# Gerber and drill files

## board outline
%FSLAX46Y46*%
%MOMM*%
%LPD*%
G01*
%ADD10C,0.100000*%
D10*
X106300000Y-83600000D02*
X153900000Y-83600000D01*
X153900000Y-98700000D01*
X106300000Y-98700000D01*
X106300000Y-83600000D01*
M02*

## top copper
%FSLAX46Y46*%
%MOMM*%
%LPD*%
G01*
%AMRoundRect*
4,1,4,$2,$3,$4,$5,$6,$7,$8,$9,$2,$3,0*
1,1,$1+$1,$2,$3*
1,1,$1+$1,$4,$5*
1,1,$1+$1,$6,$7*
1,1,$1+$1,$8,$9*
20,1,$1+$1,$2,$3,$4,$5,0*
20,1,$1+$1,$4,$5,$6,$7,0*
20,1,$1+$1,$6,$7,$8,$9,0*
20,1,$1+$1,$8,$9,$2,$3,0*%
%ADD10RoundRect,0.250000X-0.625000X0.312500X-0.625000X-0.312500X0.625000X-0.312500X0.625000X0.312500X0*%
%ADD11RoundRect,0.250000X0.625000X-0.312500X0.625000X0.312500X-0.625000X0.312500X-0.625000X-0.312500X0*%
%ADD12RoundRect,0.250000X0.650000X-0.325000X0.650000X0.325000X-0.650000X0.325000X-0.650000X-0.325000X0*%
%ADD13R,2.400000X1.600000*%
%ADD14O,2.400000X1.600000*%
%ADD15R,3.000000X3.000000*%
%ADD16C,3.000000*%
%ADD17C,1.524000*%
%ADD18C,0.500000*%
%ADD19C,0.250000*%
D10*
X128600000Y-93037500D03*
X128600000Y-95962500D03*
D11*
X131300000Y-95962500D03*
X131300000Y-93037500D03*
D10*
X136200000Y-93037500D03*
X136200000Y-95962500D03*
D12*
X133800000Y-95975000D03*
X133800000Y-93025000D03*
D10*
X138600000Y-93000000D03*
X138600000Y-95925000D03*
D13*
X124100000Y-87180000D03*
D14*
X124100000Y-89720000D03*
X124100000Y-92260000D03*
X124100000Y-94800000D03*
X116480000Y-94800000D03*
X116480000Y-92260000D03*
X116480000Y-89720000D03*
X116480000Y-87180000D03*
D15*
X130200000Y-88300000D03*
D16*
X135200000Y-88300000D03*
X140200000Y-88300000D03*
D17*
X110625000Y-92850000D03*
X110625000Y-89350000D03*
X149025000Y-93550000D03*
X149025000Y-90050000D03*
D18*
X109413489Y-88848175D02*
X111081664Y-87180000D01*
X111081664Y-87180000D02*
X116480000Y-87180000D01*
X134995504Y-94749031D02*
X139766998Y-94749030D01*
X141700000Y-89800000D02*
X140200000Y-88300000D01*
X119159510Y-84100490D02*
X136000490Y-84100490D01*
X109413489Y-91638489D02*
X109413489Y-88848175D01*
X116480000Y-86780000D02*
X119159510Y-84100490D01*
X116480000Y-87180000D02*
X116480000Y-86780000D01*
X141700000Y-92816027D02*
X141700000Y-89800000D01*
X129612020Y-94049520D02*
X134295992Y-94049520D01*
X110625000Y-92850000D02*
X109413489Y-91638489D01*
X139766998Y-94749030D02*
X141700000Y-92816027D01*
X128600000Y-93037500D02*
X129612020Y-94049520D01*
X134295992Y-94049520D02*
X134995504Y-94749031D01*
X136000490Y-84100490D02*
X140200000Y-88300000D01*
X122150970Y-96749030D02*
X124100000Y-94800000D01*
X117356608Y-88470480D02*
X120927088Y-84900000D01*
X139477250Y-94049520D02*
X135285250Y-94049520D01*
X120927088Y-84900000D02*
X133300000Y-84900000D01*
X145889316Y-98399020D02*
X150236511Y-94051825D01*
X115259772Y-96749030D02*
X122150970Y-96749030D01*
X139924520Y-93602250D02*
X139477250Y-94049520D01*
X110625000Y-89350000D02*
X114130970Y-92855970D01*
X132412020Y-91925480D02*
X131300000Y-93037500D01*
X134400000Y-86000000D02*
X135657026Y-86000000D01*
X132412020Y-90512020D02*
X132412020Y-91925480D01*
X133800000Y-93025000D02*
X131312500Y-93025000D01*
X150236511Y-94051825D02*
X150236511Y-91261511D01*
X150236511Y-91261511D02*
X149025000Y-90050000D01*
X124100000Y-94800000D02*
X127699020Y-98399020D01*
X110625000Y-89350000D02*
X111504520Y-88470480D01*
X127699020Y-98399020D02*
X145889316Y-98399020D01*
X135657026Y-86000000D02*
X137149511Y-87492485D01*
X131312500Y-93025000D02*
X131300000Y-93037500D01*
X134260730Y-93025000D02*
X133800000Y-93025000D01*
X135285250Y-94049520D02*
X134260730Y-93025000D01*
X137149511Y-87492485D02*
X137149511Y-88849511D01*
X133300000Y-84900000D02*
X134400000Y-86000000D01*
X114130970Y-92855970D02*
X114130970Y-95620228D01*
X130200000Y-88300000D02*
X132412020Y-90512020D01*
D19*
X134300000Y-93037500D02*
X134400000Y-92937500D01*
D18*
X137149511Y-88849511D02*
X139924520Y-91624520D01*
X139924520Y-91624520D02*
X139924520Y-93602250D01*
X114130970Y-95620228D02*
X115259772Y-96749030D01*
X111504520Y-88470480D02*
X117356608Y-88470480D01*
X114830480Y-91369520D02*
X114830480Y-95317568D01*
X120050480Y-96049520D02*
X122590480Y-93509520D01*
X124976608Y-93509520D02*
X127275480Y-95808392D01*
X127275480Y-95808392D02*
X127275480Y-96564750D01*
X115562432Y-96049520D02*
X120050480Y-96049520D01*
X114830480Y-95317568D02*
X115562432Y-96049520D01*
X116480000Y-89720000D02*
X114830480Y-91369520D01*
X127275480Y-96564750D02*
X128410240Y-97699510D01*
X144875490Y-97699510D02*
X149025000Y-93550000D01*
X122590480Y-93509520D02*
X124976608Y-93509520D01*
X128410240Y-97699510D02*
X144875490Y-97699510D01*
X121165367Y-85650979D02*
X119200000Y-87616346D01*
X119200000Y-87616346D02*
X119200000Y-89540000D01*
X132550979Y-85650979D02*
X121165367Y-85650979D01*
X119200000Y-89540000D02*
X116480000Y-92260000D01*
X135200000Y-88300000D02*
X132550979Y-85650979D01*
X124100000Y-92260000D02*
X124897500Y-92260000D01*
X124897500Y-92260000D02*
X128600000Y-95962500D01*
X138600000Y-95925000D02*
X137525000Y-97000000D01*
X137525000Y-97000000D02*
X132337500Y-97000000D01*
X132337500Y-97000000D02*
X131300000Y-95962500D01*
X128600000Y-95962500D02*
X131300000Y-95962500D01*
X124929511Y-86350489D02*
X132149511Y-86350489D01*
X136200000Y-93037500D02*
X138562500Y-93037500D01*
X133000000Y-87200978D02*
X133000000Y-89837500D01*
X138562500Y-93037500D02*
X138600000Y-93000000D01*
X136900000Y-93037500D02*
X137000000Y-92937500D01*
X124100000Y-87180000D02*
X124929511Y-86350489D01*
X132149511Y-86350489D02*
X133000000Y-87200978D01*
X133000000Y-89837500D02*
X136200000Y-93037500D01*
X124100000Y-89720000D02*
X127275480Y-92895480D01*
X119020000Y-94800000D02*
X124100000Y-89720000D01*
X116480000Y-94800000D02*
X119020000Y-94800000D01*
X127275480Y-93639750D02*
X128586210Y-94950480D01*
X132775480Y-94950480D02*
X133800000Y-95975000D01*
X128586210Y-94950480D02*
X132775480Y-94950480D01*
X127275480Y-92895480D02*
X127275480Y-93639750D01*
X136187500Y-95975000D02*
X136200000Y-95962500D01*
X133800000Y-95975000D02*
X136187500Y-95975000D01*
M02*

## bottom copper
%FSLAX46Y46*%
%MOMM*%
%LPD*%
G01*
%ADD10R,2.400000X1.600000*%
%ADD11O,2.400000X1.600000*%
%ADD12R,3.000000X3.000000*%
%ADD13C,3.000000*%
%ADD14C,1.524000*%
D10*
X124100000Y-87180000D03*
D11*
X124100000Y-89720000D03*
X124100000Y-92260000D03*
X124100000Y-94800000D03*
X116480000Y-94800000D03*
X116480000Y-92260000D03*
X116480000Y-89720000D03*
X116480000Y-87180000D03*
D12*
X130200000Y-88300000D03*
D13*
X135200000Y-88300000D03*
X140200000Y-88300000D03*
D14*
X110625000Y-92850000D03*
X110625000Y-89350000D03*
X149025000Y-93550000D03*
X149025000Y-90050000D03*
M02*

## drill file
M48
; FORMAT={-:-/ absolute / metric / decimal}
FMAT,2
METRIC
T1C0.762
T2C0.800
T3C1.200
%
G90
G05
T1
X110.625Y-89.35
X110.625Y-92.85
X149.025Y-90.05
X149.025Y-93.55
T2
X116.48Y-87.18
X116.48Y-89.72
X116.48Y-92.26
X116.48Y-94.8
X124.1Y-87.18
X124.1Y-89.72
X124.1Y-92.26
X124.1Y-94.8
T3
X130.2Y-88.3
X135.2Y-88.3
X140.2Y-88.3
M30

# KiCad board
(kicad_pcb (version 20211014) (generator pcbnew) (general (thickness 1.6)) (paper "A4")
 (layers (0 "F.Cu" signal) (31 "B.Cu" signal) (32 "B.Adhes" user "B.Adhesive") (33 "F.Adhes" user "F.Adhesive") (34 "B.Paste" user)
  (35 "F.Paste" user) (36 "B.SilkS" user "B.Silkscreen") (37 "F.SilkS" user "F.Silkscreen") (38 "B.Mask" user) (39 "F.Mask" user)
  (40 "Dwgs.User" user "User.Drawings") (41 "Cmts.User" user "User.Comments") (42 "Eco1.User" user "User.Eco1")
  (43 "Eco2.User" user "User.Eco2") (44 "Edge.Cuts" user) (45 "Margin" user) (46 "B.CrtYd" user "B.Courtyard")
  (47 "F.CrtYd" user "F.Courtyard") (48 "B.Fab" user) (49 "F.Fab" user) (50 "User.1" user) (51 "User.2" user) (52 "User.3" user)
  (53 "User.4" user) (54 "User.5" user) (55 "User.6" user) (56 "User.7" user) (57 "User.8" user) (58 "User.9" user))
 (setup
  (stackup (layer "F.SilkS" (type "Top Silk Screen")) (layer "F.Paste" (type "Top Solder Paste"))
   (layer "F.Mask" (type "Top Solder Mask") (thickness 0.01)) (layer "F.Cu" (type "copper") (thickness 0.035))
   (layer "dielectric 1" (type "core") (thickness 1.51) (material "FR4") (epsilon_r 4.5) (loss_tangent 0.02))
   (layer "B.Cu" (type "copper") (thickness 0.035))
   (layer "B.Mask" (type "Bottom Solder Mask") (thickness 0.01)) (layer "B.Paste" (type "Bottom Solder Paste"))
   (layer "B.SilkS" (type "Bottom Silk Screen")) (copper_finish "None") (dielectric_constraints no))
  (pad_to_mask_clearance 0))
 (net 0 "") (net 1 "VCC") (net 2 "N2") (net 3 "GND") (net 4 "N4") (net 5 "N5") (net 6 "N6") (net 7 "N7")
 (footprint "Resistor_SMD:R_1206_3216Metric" (layer "F.Cu") (at 128.6 94.5 -90)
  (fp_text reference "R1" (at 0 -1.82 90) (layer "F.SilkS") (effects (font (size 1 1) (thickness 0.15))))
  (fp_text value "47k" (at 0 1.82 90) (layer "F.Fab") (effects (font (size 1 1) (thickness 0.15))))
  (pad "1" smd roundrect (at -1.4625 0 270) (size 1.125 1.75) (layers "F.Cu" "F.Paste" "F.Mask") (roundrect_rratio 0.2222222222)
   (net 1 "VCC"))
  (pad "2" smd roundrect (at 1.4625 0 270) (size 1.125 1.75) (layers "F.Cu" "F.Paste" "F.Mask") (roundrect_rratio 0.2222222222) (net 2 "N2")))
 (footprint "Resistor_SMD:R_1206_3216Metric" (layer "F.Cu") (at 131.3 94.5 90)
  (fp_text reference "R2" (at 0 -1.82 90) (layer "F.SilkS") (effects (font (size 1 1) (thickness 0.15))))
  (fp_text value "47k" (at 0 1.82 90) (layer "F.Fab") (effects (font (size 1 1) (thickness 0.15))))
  (pad "1" smd roundrect (at -1.4625 0 90) (size 1.125 1.75) (layers "F.Cu" "F.Paste" "F.Mask") (roundrect_rratio 0.2222222222) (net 2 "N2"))
  (pad "2" smd roundrect (at 1.4625 0 90) (size 1.125 1.75) (layers "F.Cu" "F.Paste" "F.Mask") (roundrect_rratio 0.2222222222) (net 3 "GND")))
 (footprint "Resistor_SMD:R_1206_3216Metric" (layer "F.Cu") (at 136.2 94.5 -90)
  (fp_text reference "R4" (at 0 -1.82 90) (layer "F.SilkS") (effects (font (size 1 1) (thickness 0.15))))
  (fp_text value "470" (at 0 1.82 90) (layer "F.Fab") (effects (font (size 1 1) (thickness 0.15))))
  (pad "1" smd roundrect (at -1.4625 0 270) (size 1.125 1.75) (layers "F.Cu" "F.Paste" "F.Mask") (roundrect_rratio 0.2222222222)
   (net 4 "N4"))
  (pad "2" smd roundrect (at 1.4625 0 270) (size 1.125 1.75) (layers "F.Cu" "F.Paste" "F.Mask") (roundrect_rratio 0.2222222222) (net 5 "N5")))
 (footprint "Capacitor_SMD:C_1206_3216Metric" (layer "F.Cu") (at 133.8 94.5 90)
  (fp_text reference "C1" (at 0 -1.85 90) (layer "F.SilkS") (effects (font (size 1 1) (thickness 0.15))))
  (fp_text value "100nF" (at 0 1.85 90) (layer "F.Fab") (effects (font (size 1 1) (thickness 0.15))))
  (pad "1" smd roundrect (at -1.475 0 90) (size 1.15 1.8) (layers "F.Cu" "F.Paste" "F.Mask") (roundrect_rratio 0.2173913043) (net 5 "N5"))
  (pad "2" smd roundrect (at 1.475 0 90) (size 1.15 1.8) (layers "F.Cu" "F.Paste" "F.Mask") (roundrect_rratio 0.2173913043) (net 3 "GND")))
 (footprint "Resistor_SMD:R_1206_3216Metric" (layer "F.Cu") (at 138.6 94.4625 -90)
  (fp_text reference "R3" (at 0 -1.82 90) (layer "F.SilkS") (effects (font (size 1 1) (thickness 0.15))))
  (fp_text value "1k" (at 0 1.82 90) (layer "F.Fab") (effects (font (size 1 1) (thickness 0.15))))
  (pad "1" smd roundrect (at -1.4625 0 270) (size 1.125 1.75) (layers "F.Cu" "F.Paste" "F.Mask") (roundrect_rratio 0.2222222222)
   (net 4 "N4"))
  (pad "2" smd roundrect (at 1.4625 0 270) (size 1.125 1.75) (layers "F.Cu" "F.Paste" "F.Mask") (roundrect_rratio 0.2222222222) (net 2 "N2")))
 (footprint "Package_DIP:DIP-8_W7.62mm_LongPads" (layer "B.Cu") (at 124.1 87.18 180)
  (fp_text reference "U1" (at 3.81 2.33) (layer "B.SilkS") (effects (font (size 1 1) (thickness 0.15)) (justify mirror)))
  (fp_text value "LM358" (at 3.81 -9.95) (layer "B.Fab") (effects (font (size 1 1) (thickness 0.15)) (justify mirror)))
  (pad "1" thru_hole rect (at 0 0 180) (size 2.4 1.6) (drill 0.8) (layers *.Cu *.Mask) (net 4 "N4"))
  (pad "2" thru_hole oval (at 0 -2.54 180) (size 2.4 1.6) (drill 0.8) (layers *.Cu *.Mask) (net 5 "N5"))
  (pad "3" thru_hole oval (at 0 -5.08 180) (size 2.4 1.6) (drill 0.8) (layers *.Cu *.Mask) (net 2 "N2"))
  (pad "4" thru_hole oval (at 0 -7.62 180) (size 2.4 1.6) (drill 0.8) (layers *.Cu *.Mask) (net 3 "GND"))
  (pad "5" thru_hole oval (at 7.62 -7.62 180) (size 2.4 1.6) (drill 0.8) (layers *.Cu *.Mask) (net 5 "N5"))
  (pad "6" thru_hole oval (at 7.62 -5.08 180) (size 2.4 1.6) (drill 0.8) (layers *.Cu *.Mask) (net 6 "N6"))
  (pad "7" thru_hole oval (at 7.62 -2.54 180) (size 2.4 1.6) (drill 0.8) (layers *.Cu *.Mask) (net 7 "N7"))
  (pad "8" thru_hole oval (at 7.62 0 180) (size 2.4 1.6) (drill 0.8) (layers *.Cu *.Mask) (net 1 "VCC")))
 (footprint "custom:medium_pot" (layer "B.Cu") (at 130.2 88.3 -90)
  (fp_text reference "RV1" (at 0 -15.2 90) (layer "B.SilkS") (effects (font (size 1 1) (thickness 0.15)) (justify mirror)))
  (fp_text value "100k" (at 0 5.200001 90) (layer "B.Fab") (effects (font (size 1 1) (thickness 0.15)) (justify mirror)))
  (pad "1" thru_hole rect (at 0 0 90) (size 3 3) (drill 1.2) (layers *.Cu *.Mask) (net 3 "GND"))
  (pad "2" thru_hole circle (at 0 -5 90) (size 3 3) (drill 1.2) (layers *.Cu *.Mask) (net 6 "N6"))
  (pad "3" thru_hole circle (at 0 -10 90) (size 3 3) (drill 1.2) (layers *.Cu *.Mask) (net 1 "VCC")))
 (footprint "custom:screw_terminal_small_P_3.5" (layer "B.Cu") (at 115.705 91.1 90)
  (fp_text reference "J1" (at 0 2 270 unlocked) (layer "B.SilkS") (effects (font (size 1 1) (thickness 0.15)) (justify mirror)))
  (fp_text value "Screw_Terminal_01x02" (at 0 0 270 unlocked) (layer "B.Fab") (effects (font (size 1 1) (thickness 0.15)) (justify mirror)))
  (pad "1" thru_hole circle (at -1.75 -5.08 90) (size 1.524 1.524) (drill 0.762) (layers *.Cu *.Mask) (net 1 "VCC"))
  (pad "2" thru_hole circle (at 1.75 -5.08) (size 1.524 1.524) (drill 0.762) (layers *.Cu *.Mask) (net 3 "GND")))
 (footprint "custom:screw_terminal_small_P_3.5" (layer "B.Cu") (at 154.105 91.8 90)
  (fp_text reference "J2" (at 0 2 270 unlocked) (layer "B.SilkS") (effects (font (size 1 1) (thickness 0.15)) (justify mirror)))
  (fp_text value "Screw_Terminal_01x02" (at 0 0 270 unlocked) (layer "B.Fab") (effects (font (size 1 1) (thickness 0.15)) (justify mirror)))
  (pad "1" thru_hole circle (at -1.75 -5.08 90) (size 1.524 1.524) (drill 0.762) (layers *.Cu *.Mask) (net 7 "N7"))
  (pad "2" thru_hole circle (at 1.75 -5.08) (size 1.524 1.524) (drill 0.762) (layers *.Cu *.Mask) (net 3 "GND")))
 (gr_rect (start 106.3 83.6) (end 153.9 98.7) (layer "Edge.Cuts") (width 0.1) (fill none))
 (segment (start 109.413489 88.848175) (end 111.081664 87.18) (width 0.5) (layer "F.Cu") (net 1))
 (segment (start 111.081664 87.18) (end 116.48 87.18) (width 0.5) (layer "F.Cu") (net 1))
 (segment (start 134.995504 94.749031) (end 139.766998 94.74903) (width 0.5) (layer "F.Cu") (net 1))
 (segment (start 141.7 89.8) (end 140.2 88.3) (width 0.5) (layer "F.Cu") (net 1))
 (segment (start 119.15951 84.10049) (end 136.00049 84.10049) (width 0.5) (layer "F.Cu") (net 1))
 (segment (start 109.413489 91.638489) (end 109.413489 88.848175) (width 0.5) (layer "F.Cu") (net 1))
 (segment (start 116.48 86.78) (end 119.15951 84.10049) (width 0.5) (layer "F.Cu") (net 1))
 (segment (start 116.48 87.18) (end 116.48 86.78) (width 0.5) (layer "F.Cu") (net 1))
 (segment (start 141.7 92.816027) (end 141.7 89.8) (width 0.5) (layer "F.Cu") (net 1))
 (segment (start 129.61202 94.04952) (end 134.295992 94.04952) (width 0.5) (layer "F.Cu") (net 1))
 (segment (start 110.625 92.85) (end 109.413489 91.638489) (width 0.5) (layer "F.Cu") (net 1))
 (segment (start 139.766998 94.74903) (end 141.7 92.816027) (width 0.5) (layer "F.Cu") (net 1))
 (segment (start 128.6 93.0375) (end 129.61202 94.04952) (width 0.5) (layer "F.Cu") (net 1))
 (segment (start 134.295992 94.04952) (end 134.995504 94.749031) (width 0.5) (layer "F.Cu") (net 1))
 (segment (start 136.00049 84.10049) (end 140.2 88.3) (width 0.5) (layer "F.Cu") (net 1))
 (segment (start 122.15097 96.74903) (end 124.1 94.8) (width 0.5) (layer "F.Cu") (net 3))
 (segment (start 117.356608 88.47048) (end 120.927088 84.9) (width 0.5) (layer "F.Cu") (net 3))
 (segment (start 139.47725 94.04952) (end 135.28525 94.04952) (width 0.5) (layer "F.Cu") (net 3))
 (segment (start 120.927088 84.9) (end 133.3 84.9) (width 0.5) (layer "F.Cu") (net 3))
 (segment (start 145.889316 98.39902) (end 150.236511 94.051825) (width 0.5) (layer "F.Cu") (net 3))
 (segment (start 115.259772 96.74903) (end 122.15097 96.74903) (width 0.5) (layer "F.Cu") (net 3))
 (segment (start 139.92452 93.60225) (end 139.47725 94.04952) (width 0.5) (layer "F.Cu") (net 3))
 (segment (start 110.625 89.35) (end 114.13097 92.85597) (width 0.5) (layer "F.Cu") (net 3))
 (segment (start 132.41202 91.92548) (end 131.3 93.0375) (width 0.5) (layer "F.Cu") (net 3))
 (segment (start 134.4 86) (end 135.657026 86) (width 0.5) (layer "F.Cu") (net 3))
 (segment (start 132.41202 90.51202) (end 132.41202 91.92548) (width 0.5) (layer "F.Cu") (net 3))
 (segment (start 133.8 93.025) (end 131.3125 93.025) (width 0.5) (layer "F.Cu") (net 3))
 (segment (start 150.236511 94.051825) (end 150.236511 91.261511) (width 0.5) (layer "F.Cu") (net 3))
 (segment (start 150.236511 91.261511) (end 149.025 90.05) (width 0.5) (layer "F.Cu") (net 3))
 (segment (start 124.1 94.8) (end 127.69902 98.39902) (width 0.5) (layer "F.Cu") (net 3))
 (segment (start 110.625 89.35) (end 111.50452 88.47048) (width 0.5) (layer "F.Cu") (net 3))
 (segment (start 127.69902 98.39902) (end 145.889316 98.39902) (width 0.5) (layer "F.Cu") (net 3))
 (segment (start 135.657026 86) (end 137.149511 87.492485) (width 0.5) (layer "F.Cu") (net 3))
 (segment (start 131.3125 93.025) (end 131.3 93.0375) (width 0.5) (layer "F.Cu") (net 3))
 (segment (start 134.26073 93.025) (end 133.8 93.025) (width 0.5) (layer "F.Cu") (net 3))
 (segment (start 135.28525 94.04952) (end 134.26073 93.025) (width 0.5) (layer "F.Cu") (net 3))
 (segment (start 137.149511 87.492485) (end 137.149511 88.849511) (width 0.5) (layer "F.Cu") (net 3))
 (segment (start 133.3 84.9) (end 134.4 86) (width 0.5) (layer "F.Cu") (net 3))
 (segment (start 114.13097 92.85597) (end 114.13097 95.620228) (width 0.5) (layer "F.Cu") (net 3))
 (segment (start 130.2 88.3) (end 132.41202 90.51202) (width 0.5) (layer "F.Cu") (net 3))
 (segment (start 134.3 93.0375) (end 134.4 92.9375) (width 0.25) (layer "F.Cu") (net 3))
 (segment (start 137.149511 88.849511) (end 139.92452 91.62452) (width 0.5) (layer "F.Cu") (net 3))
 (segment (start 139.92452 91.62452) (end 139.92452 93.60225) (width 0.5) (layer "F.Cu") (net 3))
 (segment (start 114.13097 95.620228) (end 115.259772 96.74903) (width 0.5) (layer "F.Cu") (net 3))
 (segment (start 111.50452 88.47048) (end 117.356608 88.47048) (width 0.5) (layer "F.Cu") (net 3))
 (segment (start 114.83048 91.36952) (end 114.83048 95.317568) (width 0.5) (layer "F.Cu") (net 7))
 (segment (start 120.05048 96.04952) (end 122.59048 93.50952) (width 0.5) (layer "F.Cu") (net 7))
 (segment (start 124.976608 93.50952) (end 127.27548 95.808392) (width 0.5) (layer "F.Cu") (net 7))
 (segment (start 127.27548 95.808392) (end 127.27548 96.56475) (width 0.5) (layer "F.Cu") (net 7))
 (segment (start 115.562432 96.04952) (end 120.05048 96.04952) (width 0.5) (layer "F.Cu") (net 7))
 (segment (start 114.83048 95.317568) (end 115.562432 96.04952) (width 0.5) (layer "F.Cu") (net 7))
 (segment (start 116.48 89.72) (end 114.83048 91.36952) (width 0.5) (layer "F.Cu") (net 7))
 (segment (start 127.27548 96.56475) (end 128.41024 97.69951) (width 0.5) (layer "F.Cu") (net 7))
 (segment (start 144.87549 97.69951) (end 149.025 93.55) (width 0.5) (layer "F.Cu") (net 7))
 (segment (start 122.59048 93.50952) (end 124.976608 93.50952) (width 0.5) (layer "F.Cu") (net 7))
 (segment (start 128.41024 97.69951) (end 144.87549 97.69951) (width 0.5) (layer "F.Cu") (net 7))
 (segment (start 121.165367 85.650979) (end 119.2 87.616346) (width 0.5) (layer "F.Cu") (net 6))
 (segment (start 119.2 87.616346) (end 119.2 89.54) (width 0.5) (layer "F.Cu") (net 6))
 (segment (start 132.550979 85.650979) (end 121.165367 85.650979) (width 0.5) (layer "F.Cu") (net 6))
 (segment (start 119.2 89.54) (end 116.48 92.26) (width 0.5) (layer "F.Cu") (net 6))
 (segment (start 135.2 88.3) (end 132.550979 85.650979) (width 0.5) (layer "F.Cu") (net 6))
 (segment (start 124.1 92.26) (end 124.8975 92.26) (width 0.5) (layer "F.Cu") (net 2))
 (segment (start 124.8975 92.26) (end 128.6 95.9625) (width 0.5) (layer "F.Cu") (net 2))
 (segment (start 138.6 95.925) (end 137.525 97) (width 0.5) (layer "F.Cu") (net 2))
 (segment (start 137.525 97) (end 132.3375 97) (width 0.5) (layer "F.Cu") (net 2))
 (segment (start 132.3375 97) (end 131.3 95.9625) (width 0.5) (layer "F.Cu") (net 2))
 (segment (start 128.6 95.9625) (end 131.3 95.9625) (width 0.5) (layer "F.Cu") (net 2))
 (segment (start 124.929511 86.350489) (end 132.149511 86.350489) (width 0.5) (layer "F.Cu") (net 4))
 (segment (start 136.2 93.0375) (end 138.5625 93.0375) (width 0.5) (layer "F.Cu") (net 4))
 (segment (start 133 87.200978) (end 133 89.8375) (width 0.5) (layer "F.Cu") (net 4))
 (segment (start 138.5625 93.0375) (end 138.6 93) (width 0.5) (layer "F.Cu") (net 4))
 (segment (start 136.9 93.0375) (end 137 92.9375) (width 0.5) (layer "F.Cu") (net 4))
 (segment (start 124.1 87.18) (end 124.929511 86.350489) (width 0.5) (layer "F.Cu") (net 4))
 (segment (start 132.149511 86.350489) (end 133 87.200978) (width 0.5) (layer "F.Cu") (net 4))
 (segment (start 133 89.8375) (end 136.2 93.0375) (width 0.5) (layer "F.Cu") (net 4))
 (segment (start 124.1 89.72) (end 127.27548 92.89548) (width 0.5) (layer "F.Cu") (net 5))
 (segment (start 119.02 94.8) (end 124.1 89.72) (width 0.5) (layer "F.Cu") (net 5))
 (segment (start 116.48 94.8) (end 119.02 94.8) (width 0.5) (layer "F.Cu") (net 5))
 (segment (start 127.27548 93.63975) (end 128.58621 94.95048) (width 0.5) (layer "F.Cu") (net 5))
 (segment (start 132.77548 94.95048) (end 133.8 95.975) (width 0.5) (layer "F.Cu") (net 5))
 (segment (start 128.58621 94.95048) (end 132.77548 94.95048) (width 0.5) (layer "F.Cu") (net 5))
 (segment (start 127.27548 92.89548) (end 127.27548 93.63975) (width 0.5) (layer "F.Cu") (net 5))
 (segment (start 136.1875 95.975) (end 136.2 95.9625) (width 0.5) (layer "F.Cu") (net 5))
 (segment (start 133.8 95.975) (end 136.1875 95.975) (width 0.5) (layer "F.Cu") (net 5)))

